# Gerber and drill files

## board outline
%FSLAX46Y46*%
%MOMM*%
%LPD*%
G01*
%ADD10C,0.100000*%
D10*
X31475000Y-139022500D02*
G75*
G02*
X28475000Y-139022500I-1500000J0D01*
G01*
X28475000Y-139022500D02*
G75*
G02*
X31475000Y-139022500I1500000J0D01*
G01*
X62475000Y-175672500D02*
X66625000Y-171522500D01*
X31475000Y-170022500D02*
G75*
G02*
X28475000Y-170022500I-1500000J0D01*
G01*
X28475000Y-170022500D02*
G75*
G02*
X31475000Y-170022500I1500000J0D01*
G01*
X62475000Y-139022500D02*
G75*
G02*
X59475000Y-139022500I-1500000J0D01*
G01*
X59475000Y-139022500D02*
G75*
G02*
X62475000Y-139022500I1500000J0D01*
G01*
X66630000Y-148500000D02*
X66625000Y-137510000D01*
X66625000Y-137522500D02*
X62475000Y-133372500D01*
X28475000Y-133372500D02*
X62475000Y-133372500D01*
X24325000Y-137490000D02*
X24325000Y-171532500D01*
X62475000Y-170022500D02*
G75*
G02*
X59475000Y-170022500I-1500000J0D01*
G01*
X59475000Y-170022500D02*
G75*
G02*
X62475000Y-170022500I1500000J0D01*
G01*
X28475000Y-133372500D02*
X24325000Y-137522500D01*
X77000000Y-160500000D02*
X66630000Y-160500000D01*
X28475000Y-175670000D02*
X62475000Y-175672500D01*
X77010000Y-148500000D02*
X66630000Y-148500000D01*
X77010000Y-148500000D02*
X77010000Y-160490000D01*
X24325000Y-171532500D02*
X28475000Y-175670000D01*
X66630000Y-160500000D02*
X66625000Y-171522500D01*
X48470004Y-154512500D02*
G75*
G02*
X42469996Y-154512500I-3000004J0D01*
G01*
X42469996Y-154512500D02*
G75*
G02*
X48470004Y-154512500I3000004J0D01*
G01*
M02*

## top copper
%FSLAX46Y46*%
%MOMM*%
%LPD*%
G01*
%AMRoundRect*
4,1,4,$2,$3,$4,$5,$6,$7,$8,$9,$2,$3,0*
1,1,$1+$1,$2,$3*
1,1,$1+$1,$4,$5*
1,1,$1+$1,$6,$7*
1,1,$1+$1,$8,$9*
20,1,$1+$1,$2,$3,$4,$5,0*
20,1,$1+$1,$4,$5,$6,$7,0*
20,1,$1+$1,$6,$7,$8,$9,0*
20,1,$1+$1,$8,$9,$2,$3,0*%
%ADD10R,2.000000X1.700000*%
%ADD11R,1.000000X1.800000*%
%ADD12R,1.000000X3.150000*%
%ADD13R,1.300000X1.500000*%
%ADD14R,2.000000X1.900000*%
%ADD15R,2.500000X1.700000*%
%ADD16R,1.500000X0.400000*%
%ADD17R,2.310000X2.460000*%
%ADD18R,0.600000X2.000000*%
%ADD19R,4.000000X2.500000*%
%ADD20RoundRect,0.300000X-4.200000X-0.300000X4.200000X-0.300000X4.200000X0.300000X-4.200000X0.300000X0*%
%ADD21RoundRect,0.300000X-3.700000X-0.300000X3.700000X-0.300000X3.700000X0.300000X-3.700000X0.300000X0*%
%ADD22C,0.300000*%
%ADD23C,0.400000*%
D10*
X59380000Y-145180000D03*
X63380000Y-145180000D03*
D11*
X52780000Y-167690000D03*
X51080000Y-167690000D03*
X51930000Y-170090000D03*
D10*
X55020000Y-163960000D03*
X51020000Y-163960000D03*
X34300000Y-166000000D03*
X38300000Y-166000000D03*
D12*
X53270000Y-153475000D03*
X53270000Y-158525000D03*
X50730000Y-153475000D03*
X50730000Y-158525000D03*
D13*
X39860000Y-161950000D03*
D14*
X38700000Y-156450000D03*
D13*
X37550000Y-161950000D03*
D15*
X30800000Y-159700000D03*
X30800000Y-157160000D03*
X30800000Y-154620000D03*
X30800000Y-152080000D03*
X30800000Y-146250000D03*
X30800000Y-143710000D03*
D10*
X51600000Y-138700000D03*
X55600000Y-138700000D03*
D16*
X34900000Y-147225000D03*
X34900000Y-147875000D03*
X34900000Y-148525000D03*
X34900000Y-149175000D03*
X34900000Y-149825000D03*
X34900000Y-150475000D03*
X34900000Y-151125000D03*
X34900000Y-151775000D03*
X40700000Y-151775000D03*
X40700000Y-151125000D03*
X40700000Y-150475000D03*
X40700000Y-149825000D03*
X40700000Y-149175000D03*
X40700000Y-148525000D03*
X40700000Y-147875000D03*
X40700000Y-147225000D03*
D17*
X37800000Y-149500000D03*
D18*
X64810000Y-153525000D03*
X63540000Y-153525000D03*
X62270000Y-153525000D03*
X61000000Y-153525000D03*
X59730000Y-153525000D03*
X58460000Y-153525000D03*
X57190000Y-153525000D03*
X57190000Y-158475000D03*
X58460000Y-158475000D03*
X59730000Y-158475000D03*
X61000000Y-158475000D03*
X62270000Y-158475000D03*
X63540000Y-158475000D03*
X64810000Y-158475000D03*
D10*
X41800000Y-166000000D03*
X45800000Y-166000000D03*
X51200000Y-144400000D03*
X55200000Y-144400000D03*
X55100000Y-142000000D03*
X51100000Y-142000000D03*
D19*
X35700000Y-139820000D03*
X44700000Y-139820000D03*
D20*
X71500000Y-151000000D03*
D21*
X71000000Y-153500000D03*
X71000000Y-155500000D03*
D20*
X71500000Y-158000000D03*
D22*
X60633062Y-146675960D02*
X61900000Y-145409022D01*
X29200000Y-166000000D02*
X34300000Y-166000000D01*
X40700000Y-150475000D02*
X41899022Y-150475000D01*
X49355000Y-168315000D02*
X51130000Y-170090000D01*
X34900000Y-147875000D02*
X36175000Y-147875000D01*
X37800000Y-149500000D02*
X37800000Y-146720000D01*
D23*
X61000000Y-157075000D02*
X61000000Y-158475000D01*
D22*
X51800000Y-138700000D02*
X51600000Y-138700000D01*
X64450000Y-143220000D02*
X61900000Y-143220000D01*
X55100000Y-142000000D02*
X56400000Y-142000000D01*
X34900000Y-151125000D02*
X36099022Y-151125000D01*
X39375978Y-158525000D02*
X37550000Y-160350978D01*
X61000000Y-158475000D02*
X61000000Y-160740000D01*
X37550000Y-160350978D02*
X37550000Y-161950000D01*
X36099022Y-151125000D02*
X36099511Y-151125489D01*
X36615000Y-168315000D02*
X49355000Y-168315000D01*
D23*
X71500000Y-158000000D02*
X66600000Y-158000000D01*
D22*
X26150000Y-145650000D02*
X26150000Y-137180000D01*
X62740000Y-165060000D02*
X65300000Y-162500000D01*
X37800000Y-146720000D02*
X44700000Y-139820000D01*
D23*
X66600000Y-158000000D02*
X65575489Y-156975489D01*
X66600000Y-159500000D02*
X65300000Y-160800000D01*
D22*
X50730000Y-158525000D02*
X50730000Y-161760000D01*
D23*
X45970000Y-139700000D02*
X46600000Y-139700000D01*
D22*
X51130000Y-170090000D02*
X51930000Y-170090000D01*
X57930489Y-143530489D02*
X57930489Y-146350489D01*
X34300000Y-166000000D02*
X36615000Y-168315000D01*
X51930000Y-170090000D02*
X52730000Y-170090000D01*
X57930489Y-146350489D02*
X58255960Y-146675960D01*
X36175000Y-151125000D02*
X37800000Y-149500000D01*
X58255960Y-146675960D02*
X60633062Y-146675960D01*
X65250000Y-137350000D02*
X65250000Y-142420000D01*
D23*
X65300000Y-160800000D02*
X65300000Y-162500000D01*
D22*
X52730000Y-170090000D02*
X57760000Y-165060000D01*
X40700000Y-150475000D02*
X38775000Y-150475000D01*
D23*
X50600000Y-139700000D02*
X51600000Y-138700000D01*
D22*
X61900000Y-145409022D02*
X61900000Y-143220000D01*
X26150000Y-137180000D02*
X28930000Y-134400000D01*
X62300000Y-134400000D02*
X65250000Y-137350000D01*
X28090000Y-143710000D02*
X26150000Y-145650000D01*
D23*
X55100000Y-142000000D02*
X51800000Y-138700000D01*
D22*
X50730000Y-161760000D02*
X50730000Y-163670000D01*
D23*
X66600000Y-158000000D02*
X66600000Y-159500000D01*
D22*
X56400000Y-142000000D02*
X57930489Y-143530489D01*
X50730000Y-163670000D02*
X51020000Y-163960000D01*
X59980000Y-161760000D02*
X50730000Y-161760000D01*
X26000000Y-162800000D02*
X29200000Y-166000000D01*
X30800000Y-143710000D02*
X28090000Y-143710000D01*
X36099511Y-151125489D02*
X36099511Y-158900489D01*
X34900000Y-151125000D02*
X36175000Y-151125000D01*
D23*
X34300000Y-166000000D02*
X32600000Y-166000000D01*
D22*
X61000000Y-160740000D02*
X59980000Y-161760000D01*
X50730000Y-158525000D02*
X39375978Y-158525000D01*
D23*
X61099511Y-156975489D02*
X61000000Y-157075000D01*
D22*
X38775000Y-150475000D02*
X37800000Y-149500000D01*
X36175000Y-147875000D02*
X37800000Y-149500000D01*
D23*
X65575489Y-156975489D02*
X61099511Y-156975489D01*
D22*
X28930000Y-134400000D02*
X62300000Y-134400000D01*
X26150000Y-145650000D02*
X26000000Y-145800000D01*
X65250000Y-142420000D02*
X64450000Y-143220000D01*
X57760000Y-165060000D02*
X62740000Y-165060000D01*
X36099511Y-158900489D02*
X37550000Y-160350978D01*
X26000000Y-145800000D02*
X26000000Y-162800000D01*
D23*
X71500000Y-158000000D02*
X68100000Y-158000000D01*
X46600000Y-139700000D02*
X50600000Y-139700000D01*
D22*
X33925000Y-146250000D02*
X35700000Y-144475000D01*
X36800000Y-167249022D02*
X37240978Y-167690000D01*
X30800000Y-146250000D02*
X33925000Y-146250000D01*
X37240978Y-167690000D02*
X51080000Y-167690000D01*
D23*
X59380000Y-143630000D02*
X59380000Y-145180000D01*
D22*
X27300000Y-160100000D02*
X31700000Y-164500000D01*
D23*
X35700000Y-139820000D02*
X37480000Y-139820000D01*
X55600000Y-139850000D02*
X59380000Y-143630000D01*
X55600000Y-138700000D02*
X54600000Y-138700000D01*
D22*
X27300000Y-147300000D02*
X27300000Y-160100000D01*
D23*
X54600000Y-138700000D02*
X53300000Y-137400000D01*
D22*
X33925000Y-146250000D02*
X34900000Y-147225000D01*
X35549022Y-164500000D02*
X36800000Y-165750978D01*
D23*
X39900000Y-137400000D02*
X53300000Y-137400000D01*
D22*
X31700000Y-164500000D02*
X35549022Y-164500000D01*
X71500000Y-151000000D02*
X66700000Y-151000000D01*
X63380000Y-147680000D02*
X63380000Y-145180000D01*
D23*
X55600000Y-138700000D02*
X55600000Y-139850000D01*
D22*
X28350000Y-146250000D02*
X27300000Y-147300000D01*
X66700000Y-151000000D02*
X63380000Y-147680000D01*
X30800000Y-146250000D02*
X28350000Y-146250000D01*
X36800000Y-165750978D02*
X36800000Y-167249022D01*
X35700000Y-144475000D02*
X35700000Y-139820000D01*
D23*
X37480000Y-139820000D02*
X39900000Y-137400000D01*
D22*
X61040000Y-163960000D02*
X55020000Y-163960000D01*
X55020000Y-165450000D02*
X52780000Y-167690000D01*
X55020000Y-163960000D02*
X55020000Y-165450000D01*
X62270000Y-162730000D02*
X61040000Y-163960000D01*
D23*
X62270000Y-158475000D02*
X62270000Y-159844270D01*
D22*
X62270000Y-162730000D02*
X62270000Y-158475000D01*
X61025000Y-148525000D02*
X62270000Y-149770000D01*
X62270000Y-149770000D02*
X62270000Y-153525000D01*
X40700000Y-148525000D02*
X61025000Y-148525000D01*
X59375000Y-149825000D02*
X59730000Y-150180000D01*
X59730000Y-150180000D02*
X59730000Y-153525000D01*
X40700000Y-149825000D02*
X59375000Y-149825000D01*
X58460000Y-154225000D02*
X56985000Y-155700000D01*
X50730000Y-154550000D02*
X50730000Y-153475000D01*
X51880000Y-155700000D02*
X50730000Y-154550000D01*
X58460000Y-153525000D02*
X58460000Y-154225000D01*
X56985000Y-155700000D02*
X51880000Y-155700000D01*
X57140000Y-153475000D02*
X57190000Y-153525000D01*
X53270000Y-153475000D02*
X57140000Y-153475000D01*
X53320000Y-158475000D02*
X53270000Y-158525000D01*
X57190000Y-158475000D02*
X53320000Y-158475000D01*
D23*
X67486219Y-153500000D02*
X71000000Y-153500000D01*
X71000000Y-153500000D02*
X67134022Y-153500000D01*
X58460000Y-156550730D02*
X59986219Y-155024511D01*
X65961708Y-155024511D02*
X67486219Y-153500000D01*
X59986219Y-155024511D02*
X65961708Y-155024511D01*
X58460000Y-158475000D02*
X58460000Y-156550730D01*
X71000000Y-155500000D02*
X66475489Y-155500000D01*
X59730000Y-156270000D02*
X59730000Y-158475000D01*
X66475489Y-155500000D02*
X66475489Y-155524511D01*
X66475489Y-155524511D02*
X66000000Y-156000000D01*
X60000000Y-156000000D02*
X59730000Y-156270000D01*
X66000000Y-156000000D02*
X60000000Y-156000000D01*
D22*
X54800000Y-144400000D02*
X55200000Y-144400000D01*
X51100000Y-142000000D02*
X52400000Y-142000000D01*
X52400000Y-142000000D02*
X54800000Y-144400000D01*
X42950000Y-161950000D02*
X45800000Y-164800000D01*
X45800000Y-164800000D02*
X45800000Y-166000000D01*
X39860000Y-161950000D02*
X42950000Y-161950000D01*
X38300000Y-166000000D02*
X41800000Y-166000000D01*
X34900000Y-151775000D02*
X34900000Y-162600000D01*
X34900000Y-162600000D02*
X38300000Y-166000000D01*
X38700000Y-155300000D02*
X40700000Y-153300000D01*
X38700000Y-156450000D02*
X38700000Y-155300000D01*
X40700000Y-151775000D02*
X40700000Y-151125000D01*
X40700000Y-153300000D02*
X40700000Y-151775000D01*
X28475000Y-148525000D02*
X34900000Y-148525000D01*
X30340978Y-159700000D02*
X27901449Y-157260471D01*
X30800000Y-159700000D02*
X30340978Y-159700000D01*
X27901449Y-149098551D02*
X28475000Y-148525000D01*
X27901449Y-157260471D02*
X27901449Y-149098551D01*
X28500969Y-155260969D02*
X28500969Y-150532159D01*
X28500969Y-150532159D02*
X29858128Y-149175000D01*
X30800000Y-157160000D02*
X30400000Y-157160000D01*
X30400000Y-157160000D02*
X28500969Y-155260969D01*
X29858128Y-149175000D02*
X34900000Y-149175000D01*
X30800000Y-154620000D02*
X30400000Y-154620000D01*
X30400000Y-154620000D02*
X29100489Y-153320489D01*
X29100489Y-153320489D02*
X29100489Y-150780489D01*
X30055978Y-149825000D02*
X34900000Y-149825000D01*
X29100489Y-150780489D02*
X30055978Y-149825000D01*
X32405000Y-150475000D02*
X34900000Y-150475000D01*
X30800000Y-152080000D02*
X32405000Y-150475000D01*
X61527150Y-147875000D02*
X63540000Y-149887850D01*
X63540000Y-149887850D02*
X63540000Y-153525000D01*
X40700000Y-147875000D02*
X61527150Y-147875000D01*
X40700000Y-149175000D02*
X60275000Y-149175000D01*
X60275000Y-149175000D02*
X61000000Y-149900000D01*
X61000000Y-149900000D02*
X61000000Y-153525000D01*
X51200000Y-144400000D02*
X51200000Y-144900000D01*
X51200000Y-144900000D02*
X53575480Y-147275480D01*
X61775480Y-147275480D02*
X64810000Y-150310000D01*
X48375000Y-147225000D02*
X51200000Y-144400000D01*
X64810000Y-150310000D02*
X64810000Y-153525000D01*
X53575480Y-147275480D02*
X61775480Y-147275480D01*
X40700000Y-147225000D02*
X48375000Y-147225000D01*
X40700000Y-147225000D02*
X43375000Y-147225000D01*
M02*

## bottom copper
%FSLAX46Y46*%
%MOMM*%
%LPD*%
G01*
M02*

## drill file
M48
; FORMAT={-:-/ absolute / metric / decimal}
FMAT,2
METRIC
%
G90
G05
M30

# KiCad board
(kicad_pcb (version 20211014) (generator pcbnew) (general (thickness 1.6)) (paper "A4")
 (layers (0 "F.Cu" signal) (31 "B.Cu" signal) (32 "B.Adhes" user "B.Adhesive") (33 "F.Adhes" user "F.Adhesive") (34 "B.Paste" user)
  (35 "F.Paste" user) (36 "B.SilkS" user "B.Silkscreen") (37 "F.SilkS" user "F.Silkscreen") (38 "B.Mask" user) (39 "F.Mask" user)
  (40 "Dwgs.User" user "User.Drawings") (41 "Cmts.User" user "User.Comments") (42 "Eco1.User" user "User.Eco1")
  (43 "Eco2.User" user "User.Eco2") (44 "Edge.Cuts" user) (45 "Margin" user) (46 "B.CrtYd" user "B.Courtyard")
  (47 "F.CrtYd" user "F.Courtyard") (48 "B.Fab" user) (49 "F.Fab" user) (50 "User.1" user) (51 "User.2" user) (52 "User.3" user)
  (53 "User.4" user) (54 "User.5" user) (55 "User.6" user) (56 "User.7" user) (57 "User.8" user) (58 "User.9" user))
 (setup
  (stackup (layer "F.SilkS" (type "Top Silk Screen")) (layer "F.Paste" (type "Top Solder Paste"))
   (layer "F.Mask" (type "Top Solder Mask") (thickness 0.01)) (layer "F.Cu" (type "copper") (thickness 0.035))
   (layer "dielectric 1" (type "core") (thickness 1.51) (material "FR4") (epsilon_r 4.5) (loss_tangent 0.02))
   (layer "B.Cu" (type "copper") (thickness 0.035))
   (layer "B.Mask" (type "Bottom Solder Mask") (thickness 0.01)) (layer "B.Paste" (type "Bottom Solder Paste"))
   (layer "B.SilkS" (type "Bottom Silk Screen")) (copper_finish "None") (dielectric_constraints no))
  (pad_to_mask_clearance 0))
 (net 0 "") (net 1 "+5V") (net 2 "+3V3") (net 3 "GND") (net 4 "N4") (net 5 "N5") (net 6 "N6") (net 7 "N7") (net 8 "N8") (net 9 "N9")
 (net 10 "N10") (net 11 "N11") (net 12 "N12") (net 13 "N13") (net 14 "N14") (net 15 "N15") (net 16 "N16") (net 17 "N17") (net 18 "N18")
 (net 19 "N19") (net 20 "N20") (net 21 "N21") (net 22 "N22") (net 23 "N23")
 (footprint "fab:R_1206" (layer "F.Cu") (at 61.38 145.18)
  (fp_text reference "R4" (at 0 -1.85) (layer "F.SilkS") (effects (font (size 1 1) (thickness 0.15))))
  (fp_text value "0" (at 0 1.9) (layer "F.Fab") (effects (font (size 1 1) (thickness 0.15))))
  (pad "1" smd rect locked (at -2 0) (size 2 1.7) (layers "F.Cu" "F.Paste" "F.Mask") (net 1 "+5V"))
  (pad "2" smd rect locked (at 2 0) (size 2 1.7) (layers "F.Cu" "F.Paste" "F.Mask") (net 1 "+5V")))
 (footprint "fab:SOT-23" (layer "F.Cu") (at 51.93 168.89 -90)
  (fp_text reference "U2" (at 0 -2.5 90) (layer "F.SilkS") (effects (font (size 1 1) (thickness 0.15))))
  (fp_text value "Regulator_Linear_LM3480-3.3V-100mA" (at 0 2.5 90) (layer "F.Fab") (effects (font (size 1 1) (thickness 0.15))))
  (pad "1" smd rect locked (at -1.2 -0.85 270) (size 1.8 1) (layers "F.Cu" "F.Paste" "F.Mask") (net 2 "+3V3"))
  (pad "2" smd rect locked (at -1.2 0.85 270) (size 1.8 1) (layers "F.Cu" "F.Paste" "F.Mask") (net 1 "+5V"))
  (pad "3" smd rect locked (at 1.2 0 270) (size 1.8 1) (layers "F.Cu" "F.Paste" "F.Mask") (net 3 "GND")))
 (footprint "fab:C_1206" (layer "F.Cu") (at 53.02 163.96 180)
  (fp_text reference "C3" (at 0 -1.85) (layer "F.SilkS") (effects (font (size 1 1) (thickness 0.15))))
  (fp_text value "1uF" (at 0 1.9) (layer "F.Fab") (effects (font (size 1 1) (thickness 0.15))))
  (pad "1" smd rect locked (at -2 0 180) (size 2 1.7) (layers "F.Cu" "F.Paste" "F.Mask") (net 2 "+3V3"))
  (pad "2" smd rect locked (at 2 0 180) (size 2 1.7) (layers "F.Cu" "F.Paste" "F.Mask") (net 3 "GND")))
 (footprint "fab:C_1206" (layer "F.Cu") (at 36.3 166)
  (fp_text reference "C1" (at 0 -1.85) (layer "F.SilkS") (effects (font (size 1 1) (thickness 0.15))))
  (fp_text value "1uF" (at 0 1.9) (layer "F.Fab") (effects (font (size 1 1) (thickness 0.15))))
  (pad "1" smd rect locked (at -2 0) (size 2 1.7) (layers "F.Cu" "F.Paste" "F.Mask") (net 3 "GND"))
  (pad "2" smd rect locked (at 2 0) (size 2 1.7) (layers "F.Cu" "F.Paste" "F.Mask") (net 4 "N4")))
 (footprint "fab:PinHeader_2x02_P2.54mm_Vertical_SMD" (layer "F.Cu") (at 52 156 -90)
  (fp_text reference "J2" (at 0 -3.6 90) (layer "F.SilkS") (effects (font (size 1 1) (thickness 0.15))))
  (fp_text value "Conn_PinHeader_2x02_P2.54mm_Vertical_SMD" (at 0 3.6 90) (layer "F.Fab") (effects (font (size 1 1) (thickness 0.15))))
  (pad "1" smd rect locked (at -2.525 -1.27 270) (size 3.15 1) (layers "F.Cu" "F.Paste" "F.Mask") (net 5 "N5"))
  (pad "2" smd rect locked (at 2.525 -1.27 270) (size 3.15 1) (layers "F.Cu" "F.Paste" "F.Mask") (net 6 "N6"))
  (pad "3" smd rect locked (at -2.525 1.27 270) (size 3.15 1) (layers "F.Cu" "F.Paste" "F.Mask") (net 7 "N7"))
  (pad "4" smd rect locked (at 2.525 1.27 270) (size 3.15 1) (layers "F.Cu" "F.Paste" "F.Mask") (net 3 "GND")))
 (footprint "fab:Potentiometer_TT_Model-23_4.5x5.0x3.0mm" (layer "F.Cu") (at 38.7 159.2)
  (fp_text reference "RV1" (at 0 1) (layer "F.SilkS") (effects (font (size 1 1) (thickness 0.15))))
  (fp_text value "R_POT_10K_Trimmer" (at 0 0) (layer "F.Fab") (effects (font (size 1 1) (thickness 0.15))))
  (pad "1" smd rect locked (at 1.16 2.75) (size 1.3 1.5) (layers "F.Cu" "F.Paste" "F.Mask") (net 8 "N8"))
  (pad "2" smd rect locked (at 0 -2.75) (size 2 1.9) (layers "F.Cu" "F.Paste" "F.Mask") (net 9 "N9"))
  (pad "3" smd rect locked (at -1.15 2.75) (size 1.3 1.5) (layers "F.Cu" "F.Paste" "F.Mask") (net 3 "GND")))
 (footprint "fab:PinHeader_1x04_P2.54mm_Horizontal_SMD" (layer "F.Cu") (at 30.8 159.7 180)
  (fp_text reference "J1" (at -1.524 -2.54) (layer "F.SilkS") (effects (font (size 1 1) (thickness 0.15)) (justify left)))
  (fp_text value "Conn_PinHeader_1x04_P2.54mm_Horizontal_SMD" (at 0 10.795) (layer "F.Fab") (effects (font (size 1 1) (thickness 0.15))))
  (pad "1" smd rect locked (at 0 0 180) (size 2.5 1.7) (layers "F.Cu" "F.Paste" "F.Mask") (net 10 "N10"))
  (pad "2" smd rect locked (at 0 2.54 180) (size 2.5 1.7) (layers "F.Cu" "F.Paste" "F.Mask") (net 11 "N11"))
  (pad "3" smd rect locked (at 0 5.08 180) (size 2.5 1.7) (layers "F.Cu" "F.Paste" "F.Mask") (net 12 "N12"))
  (pad "4" smd rect locked (at 0 7.62 180) (size 2.5 1.7) (layers "F.Cu" "F.Paste" "F.Mask") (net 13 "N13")))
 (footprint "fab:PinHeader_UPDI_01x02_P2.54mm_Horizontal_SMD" (layer "F.Cu") (at 30.8 146.25 180)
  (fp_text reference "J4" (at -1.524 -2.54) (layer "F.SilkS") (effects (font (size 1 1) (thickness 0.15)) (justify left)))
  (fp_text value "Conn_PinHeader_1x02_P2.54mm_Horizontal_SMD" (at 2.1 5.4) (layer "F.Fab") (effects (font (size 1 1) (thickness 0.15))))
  (pad "1" smd rect locked (at 0 0 180) (size 2.5 1.7) (layers "F.Cu" "F.Paste" "F.Mask") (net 1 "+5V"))
  (pad "2" smd rect locked (at 0 2.54 180) (size 2.5 1.7) (layers "F.Cu" "F.Paste" "F.Mask") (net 3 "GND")))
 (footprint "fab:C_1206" (layer "F.Cu") (at 53.6 138.7)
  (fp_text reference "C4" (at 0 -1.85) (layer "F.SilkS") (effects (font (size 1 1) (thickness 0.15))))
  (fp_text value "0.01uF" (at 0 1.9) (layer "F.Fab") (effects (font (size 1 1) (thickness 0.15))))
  (pad "1" smd rect locked (at -2 0) (size 2 1.7) (layers "F.Cu" "F.Paste" "F.Mask") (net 3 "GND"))
  (pad "2" smd rect locked (at 2 0) (size 2 1.7) (layers "F.Cu" "F.Paste" "F.Mask") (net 1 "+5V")))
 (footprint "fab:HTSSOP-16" (layer "F.Cu") (at 37.8 149.5)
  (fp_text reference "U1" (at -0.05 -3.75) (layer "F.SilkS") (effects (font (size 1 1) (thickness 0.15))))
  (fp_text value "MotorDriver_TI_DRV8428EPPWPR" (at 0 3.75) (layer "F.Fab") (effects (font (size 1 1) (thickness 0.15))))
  (pad "1" smd rect locked (at -2.9 -2.275 270) (size 0.4 1.5) (layers "F.Cu" "F.Paste" "F.Mask") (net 1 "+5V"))
  (pad "2" smd rect locked (at -2.9 -1.625 270) (size 0.4 1.5) (layers "F.Cu" "F.Paste" "F.Mask") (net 3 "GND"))
  (pad "3" smd rect locked (at -2.9 -0.975 270) (size 0.4 1.5) (layers "F.Cu" "F.Paste" "F.Mask") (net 10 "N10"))
  (pad "4" smd rect locked (at -2.9 -0.325 270) (size 0.4 1.5) (layers "F.Cu" "F.Paste" "F.Mask") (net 11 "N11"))
  (pad "5" smd rect locked (at -2.9 0.325 270) (size 0.4 1.5) (layers "F.Cu" "F.Paste" "F.Mask") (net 12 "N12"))
  (pad "6" smd rect locked (at -2.9 0.975 270) (size 0.4 1.5) (layers "F.Cu" "F.Paste" "F.Mask") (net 13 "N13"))
  (pad "7" smd rect locked (at -2.9 1.625 270) (size 0.4 1.5) (layers "F.Cu" "F.Paste" "F.Mask") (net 3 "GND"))
  (pad "8" smd rect locked (at -2.9 2.275 270) (size 0.4 1.5) (layers "F.Cu" "F.Paste" "F.Mask") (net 4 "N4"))
  (pad "9" smd rect locked (at 2.9 2.275 270) (size 0.4 1.5) (layers "F.Cu" "F.Paste" "F.Mask") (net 9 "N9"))
  (pad "10" smd rect locked (at 2.9 1.625 270) (size 0.4 1.5) (layers "F.Cu" "F.Paste" "F.Mask") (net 9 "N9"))
  (pad "11" smd rect locked (at 2.9 0.975 270) (size 0.4 1.5) (layers "F.Cu" "F.Paste" "F.Mask") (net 3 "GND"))
  (pad "12" smd rect locked (at 2.9 0.325 270) (size 0.4 1.5) (layers "F.Cu" "F.Paste" "F.Mask") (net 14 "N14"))
  (pad "13" smd rect locked (at 2.9 -0.325 270) (size 0.4 1.5) (layers "F.Cu" "F.Paste" "F.Mask") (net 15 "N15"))
  (pad "14" smd rect locked (at 2.9 -0.975 270) (size 0.4 1.5) (layers "F.Cu" "F.Paste" "F.Mask") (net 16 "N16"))
  (pad "15" smd rect locked (at 2.9 -1.625 270) (size 0.4 1.5) (layers "F.Cu" "F.Paste" "F.Mask") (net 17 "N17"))
  (pad "16" smd rect locked (at 2.9 -2.275 270) (size 0.4 1.5) (layers "F.Cu" "F.Paste" "F.Mask") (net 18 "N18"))
  (pad "17" smd rect locked (at 0 0 270) (size 2.46 2.31) (layers "F.Cu" "F.Paste" "F.Mask") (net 3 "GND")))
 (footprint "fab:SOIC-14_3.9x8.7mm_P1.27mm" (layer "F.Cu") (at 61 156 -90)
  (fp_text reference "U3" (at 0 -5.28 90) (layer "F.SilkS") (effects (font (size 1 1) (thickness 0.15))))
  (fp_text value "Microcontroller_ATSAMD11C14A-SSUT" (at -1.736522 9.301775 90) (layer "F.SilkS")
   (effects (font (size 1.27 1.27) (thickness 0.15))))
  (pad "1" smd rect locked (at -2.475 -3.81 270) (size 2 0.6) (layers "F.Cu" "F.Paste" "F.Mask") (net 18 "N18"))
  (pad "2" smd rect locked (at -2.475 -2.54 270) (size 2 0.6) (layers "F.Cu" "F.Paste" "F.Mask") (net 17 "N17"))
  (pad "3" smd rect locked (at -2.475 -1.27 270) (size 2 0.6) (layers "F.Cu" "F.Paste" "F.Mask") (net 16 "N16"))
  (pad "4" smd rect locked (at -2.475 0 270) (size 2 0.6) (layers "F.Cu" "F.Paste" "F.Mask") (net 15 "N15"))
  (pad "5" smd rect locked (at -2.475 1.27 270) (size 2 0.6) (layers "F.Cu" "F.Paste" "F.Mask") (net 14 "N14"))
  (pad "6" smd rect locked (at -2.475 2.54 270) (size 2 0.6) (layers "F.Cu" "F.Paste" "F.Mask") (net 7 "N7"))
  (pad "7" smd rect locked (at -2.475 3.81 270) (size 2 0.6) (layers "F.Cu" "F.Paste" "F.Mask") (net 5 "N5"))
  (pad "8" smd rect locked (at 2.475 3.81 270) (size 2 0.6) (layers "F.Cu" "F.Paste" "F.Mask") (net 6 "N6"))
  (pad "9" smd rect locked (at 2.475 2.54 270) (size 2 0.6) (layers "F.Cu" "F.Paste" "F.Mask") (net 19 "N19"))
  (pad "10" smd rect locked (at 2.475 1.27 270) (size 2 0.6) (layers "F.Cu" "F.Paste" "F.Mask") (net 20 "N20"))
  (pad "11" smd rect locked (at 2.475 0 270) (size 2 0.6) (layers "F.Cu" "F.Paste" "F.Mask") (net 3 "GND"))
  (pad "12" smd rect locked (at 2.475 -1.27 270) (size 2 0.6) (layers "F.Cu" "F.Paste" "F.Mask") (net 2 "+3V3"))
  (pad "13" smd rect locked (at 2.475 -2.54 270) (size 2 0.6) (layers "F.Cu" "F.Paste" "F.Mask") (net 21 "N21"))
  (pad "14" smd rect locked (at 2.475 -3.81 270) (size 2 0.6) (layers "F.Cu" "F.Paste" "F.Mask") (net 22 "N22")))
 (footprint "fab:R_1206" (layer "F.Cu") (at 43.8 166)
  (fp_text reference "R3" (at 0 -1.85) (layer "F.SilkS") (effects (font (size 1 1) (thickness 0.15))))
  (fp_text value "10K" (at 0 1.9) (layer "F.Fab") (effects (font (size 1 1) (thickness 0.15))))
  (pad "1" smd rect locked (at -2 0) (size 2 1.7) (layers "F.Cu" "F.Paste" "F.Mask") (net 4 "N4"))
  (pad "2" smd rect locked (at 2 0) (size 2 1.7) (layers "F.Cu" "F.Paste" "F.Mask") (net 8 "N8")))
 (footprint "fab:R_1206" (layer "F.Cu") (at 53.2 144.4)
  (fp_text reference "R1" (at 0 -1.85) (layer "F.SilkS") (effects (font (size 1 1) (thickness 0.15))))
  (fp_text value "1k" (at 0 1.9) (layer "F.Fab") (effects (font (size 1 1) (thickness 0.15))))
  (pad "1" smd rect locked (at -2 0) (size 2 1.7) (layers "F.Cu" "F.Paste" "F.Mask") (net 18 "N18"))
  (pad "2" smd rect locked (at 2 0) (size 2 1.7) (layers "F.Cu" "F.Paste" "F.Mask") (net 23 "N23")))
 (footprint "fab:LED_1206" (layer "F.Cu") (at 53.1 142 180)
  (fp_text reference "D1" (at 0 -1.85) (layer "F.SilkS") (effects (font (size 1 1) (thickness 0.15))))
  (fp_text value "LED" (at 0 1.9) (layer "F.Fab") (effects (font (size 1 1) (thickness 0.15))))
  (pad "1" smd rect locked (at -2 0 180) (size 2 1.7) (layers "F.Cu" "F.Paste" "F.Mask") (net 3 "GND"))
  (pad "2" smd rect locked (at 2 0 180) (size 2 1.7) (layers "F.Cu" "F.Paste" "F.Mask") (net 23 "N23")))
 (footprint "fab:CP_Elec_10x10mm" (layer "F.Cu") (at 40.2 139.82)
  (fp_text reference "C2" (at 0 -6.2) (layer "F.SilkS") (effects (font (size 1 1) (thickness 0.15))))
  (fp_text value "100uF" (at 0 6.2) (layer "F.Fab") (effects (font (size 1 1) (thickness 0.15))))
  (pad "1" smd rect locked (at -4.5 0) (size 4 2.5) (layers "F.Cu" "F.Paste" "F.Mask") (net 1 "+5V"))
  (pad "2" smd rect locked (at 4.5 0) (size 4 2.5) (layers "F.Cu" "F.Paste" "F.Mask") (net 3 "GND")))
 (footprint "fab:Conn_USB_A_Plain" (layer "F.Cu") (at 71 154.5)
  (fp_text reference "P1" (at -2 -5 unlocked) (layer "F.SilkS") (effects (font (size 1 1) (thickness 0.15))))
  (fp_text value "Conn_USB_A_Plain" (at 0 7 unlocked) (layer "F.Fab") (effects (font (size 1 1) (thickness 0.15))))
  (pad "1" smd roundrect (at 0.5 -3.5) (size 9 1.2) (layers "F.Cu" "F.Paste" "F.Mask") (roundrect_rratio 0.25) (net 1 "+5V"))
  (pad "2" smd roundrect (at 0 -1) (size 8 1.2) (layers "F.Cu" "F.Paste" "F.Mask") (roundrect_rratio 0.25) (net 19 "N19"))
  (pad "3" smd roundrect (at 0 1) (size 8 1.2) (layers "F.Cu" "F.Paste" "F.Mask") (roundrect_rratio 0.25) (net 20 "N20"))
  (pad "4" smd roundrect (at 0.5 3.5) (size 9 1.2) (layers "F.Cu" "F.Paste" "F.Mask") (roundrect_rratio 0.25) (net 3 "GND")))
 (gr_circle (center 29.975 139.0225) (end 28.475 139.0225) (layer "Edge.Cuts") (width 0.1) (fill none))
 (gr_line (start 62.475 175.6725) (end 66.625 171.5225) (layer "Edge.Cuts") (width 0.1))
 (gr_circle (center 29.975 170.0225) (end 31.475 170.0225) (layer "Edge.Cuts") (width 0.1) (fill none))
 (gr_circle (center 60.975 139.0225) (end 62.475 139.0225) (layer "Edge.Cuts") (width 0.1) (fill none))
 (gr_line (start 66.63 148.5) (end 66.625 137.51) (layer "Edge.Cuts") (width 0.1))
 (gr_line (start 66.625 137.5225) (end 62.475 133.3725) (layer "Edge.Cuts") (width 0.1))
 (gr_line (start 28.475 133.3725) (end 62.475 133.3725) (layer "Edge.Cuts") (width 0.1))
 (gr_line (start 24.325 137.49) (end 24.325 171.5325) (layer "Edge.Cuts") (width 0.1))
 (gr_circle (center 60.975 170.0225) (end 62.475 170.0225) (layer "Edge.Cuts") (width 0.1) (fill none))
 (gr_line (start 28.475 133.3725) (end 24.325 137.5225) (layer "Edge.Cuts") (width 0.1))
 (gr_line (start 77 160.5) (end 66.63 160.5) (layer "Edge.Cuts") (width 0.1))
 (gr_line (start 28.475 175.67) (end 62.475 175.6725) (layer "Edge.Cuts") (width 0.1))
 (gr_line (start 77.01 148.5) (end 66.63 148.5) (layer "Edge.Cuts") (width 0.1))
 (gr_line (start 77.01 148.5) (end 77.01 160.49) (layer "Edge.Cuts") (width 0.1))
 (gr_line (start 24.325 171.5325) (end 28.475 175.67) (layer "Edge.Cuts") (width 0.1))
 (gr_line (start 66.63 160.5) (end 66.625 171.5225) (layer "Edge.Cuts") (width 0.1))
 (gr_circle (center 45.47 154.5125) (end 45.475 151.5125) (layer "Edge.Cuts") (width 0.1) (fill none))
 (segment (start 60.633062 146.67596) (end 61.9 145.409022) (width 0.3) (layer "F.Cu") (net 3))
 (segment (start 29.2 166) (end 34.3 166) (width 0.3) (layer "F.Cu") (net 3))
 (segment (start 40.7 150.475) (end 41.899022 150.475) (width 0.3) (layer "F.Cu") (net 3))
 (segment (start 49.355 168.315) (end 51.13 170.09) (width 0.3) (layer "F.Cu") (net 3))
 (segment (start 34.9 147.875) (end 36.175 147.875) (width 0.3) (layer "F.Cu") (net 3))
 (segment (start 37.8 149.5) (end 37.8 146.72) (width 0.3) (layer "F.Cu") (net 3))
 (segment (start 61 157.075) (end 61 158.475) (width 0.4) (layer "F.Cu") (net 3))
 (segment (start 51.8 138.7) (end 51.6 138.7) (width 0.3) (layer "F.Cu") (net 3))
 (segment (start 64.45 143.22) (end 61.9 143.22) (width 0.3) (layer "F.Cu") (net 3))
 (segment (start 55.1 142) (end 56.4 142) (width 0.3) (layer "F.Cu") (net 3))
 (segment (start 34.9 151.125) (end 36.099022 151.125) (width 0.3) (layer "F.Cu") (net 3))
 (segment (start 39.375978 158.525) (end 37.55 160.350978) (width 0.3) (layer "F.Cu") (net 3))
 (segment (start 61 158.475) (end 61 160.74) (width 0.3) (layer "F.Cu") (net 3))
 (segment (start 37.55 160.350978) (end 37.55 161.95) (width 0.3) (layer "F.Cu") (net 3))
 (segment (start 36.099022 151.125) (end 36.099511 151.125489) (width 0.3) (layer "F.Cu") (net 3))
 (segment (start 36.615 168.315) (end 49.355 168.315) (width 0.3) (layer "F.Cu") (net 3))
 (segment (start 71.5 158) (end 66.6 158) (width 0.4) (layer "F.Cu") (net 3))
 (segment (start 26.15 145.65) (end 26.15 137.18) (width 0.3) (layer "F.Cu") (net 3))
 (segment (start 62.74 165.06) (end 65.3 162.5) (width 0.3) (layer "F.Cu") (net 3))
 (segment (start 37.8 146.72) (end 44.7 139.82) (width 0.3) (layer "F.Cu") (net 3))
 (segment (start 66.6 158) (end 65.575489 156.975489) (width 0.4) (layer "F.Cu") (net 3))
 (segment (start 66.6 159.5) (end 65.3 160.8) (width 0.4) (layer "F.Cu") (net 3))
 (segment (start 50.73 158.525) (end 50.73 161.76) (width 0.3) (layer "F.Cu") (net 3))
 (segment (start 45.97 139.7) (end 46.6 139.7) (width 0.4) (layer "F.Cu") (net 3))
 (segment (start 51.13 170.09) (end 51.93 170.09) (width 0.3) (layer "F.Cu") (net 3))
 (segment (start 57.930489 143.530489) (end 57.930489 146.350489) (width 0.3) (layer "F.Cu") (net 3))
 (segment (start 34.3 166) (end 36.615 168.315) (width 0.3) (layer "F.Cu") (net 3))
 (segment (start 51.93 170.09) (end 52.73 170.09) (width 0.3) (layer "F.Cu") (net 3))
 (segment (start 57.930489 146.350489) (end 58.25596 146.67596) (width 0.3) (layer "F.Cu") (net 3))
 (segment (start 36.175 151.125) (end 37.8 149.5) (width 0.3) (layer "F.Cu") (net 3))
 (segment (start 58.25596 146.67596) (end 60.633062 146.67596) (width 0.3) (layer "F.Cu") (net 3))
 (segment (start 65.25 137.35) (end 65.25 142.42) (width 0.3) (layer "F.Cu") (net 3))
 (segment (start 65.3 160.8) (end 65.3 162.5) (width 0.4) (layer "F.Cu") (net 3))
 (segment (start 52.73 170.09) (end 57.76 165.06) (width 0.3) (layer "F.Cu") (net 3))
 (segment (start 40.7 150.475) (end 38.775 150.475) (width 0.3) (layer "F.Cu") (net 3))
 (segment (start 50.6 139.7) (end 51.6 138.7) (width 0.4) (layer "F.Cu") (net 3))
 (segment (start 61.9 145.409022) (end 61.9 143.22) (width 0.3) (layer "F.Cu") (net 3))
 (segment (start 26.15 137.18) (end 28.93 134.4) (width 0.3) (layer "F.Cu") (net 3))
 (segment (start 62.3 134.4) (end 65.25 137.35) (width 0.3) (layer "F.Cu") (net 3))
 (segment (start 28.09 143.71) (end 26.15 145.65) (width 0.3) (layer "F.Cu") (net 3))
 (segment (start 55.1 142) (end 51.8 138.7) (width 0.4) (layer "F.Cu") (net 3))
 (segment (start 50.73 161.76) (end 50.73 163.67) (width 0.3) (layer "F.Cu") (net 3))
 (segment (start 66.6 158) (end 66.6 159.5) (width 0.4) (layer "F.Cu") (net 3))
 (segment (start 56.4 142) (end 57.930489 143.530489) (width 0.3) (layer "F.Cu") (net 3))
 (segment (start 50.73 163.67) (end 51.02 163.96) (width 0.3) (layer "F.Cu") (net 3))
 (segment (start 59.98 161.76) (end 50.73 161.76) (width 0.3) (layer "F.Cu") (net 3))
 (segment (start 26 162.8) (end 29.2 166) (width 0.3) (layer "F.Cu") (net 3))
 (segment (start 30.8 143.71) (end 28.09 143.71) (width 0.3) (layer "F.Cu") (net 3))
 (segment (start 36.099511 151.125489) (end 36.099511 158.900489) (width 0.3) (layer "F.Cu") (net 3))
 (segment (start 34.9 151.125) (end 36.175 151.125) (width 0.3) (layer "F.Cu") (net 3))
 (segment (start 34.3 166) (end 32.6 166) (width 0.4) (layer "F.Cu") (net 3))
 (segment (start 61 160.74) (end 59.98 161.76) (width 0.3) (layer "F.Cu") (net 3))
 (segment (start 50.73 158.525) (end 39.375978 158.525) (width 0.3) (layer "F.Cu") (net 3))
 (segment (start 61.099511 156.975489) (end 61 157.075) (width 0.4) (layer "F.Cu") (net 3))
 (segment (start 38.775 150.475) (end 37.8 149.5) (width 0.3) (layer "F.Cu") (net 3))
 (segment (start 36.175 147.875) (end 37.8 149.5) (width 0.3) (layer "F.Cu") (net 3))
 (segment (start 65.575489 156.975489) (end 61.099511 156.975489) (width 0.4) (layer "F.Cu") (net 3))
 (segment (start 28.93 134.4) (end 62.3 134.4) (width 0.3) (layer "F.Cu") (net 3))
 (segment (start 26.15 145.65) (end 26 145.8) (width 0.3) (layer "F.Cu") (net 3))
 (segment (start 65.25 142.42) (end 64.45 143.22) (width 0.3) (layer "F.Cu") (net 3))
 (segment (start 57.76 165.06) (end 62.74 165.06) (width 0.3) (layer "F.Cu") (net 3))
 (segment (start 36.099511 158.900489) (end 37.55 160.350978) (width 0.3) (layer "F.Cu") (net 3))
 (segment (start 26 145.8) (end 26 162.8) (width 0.3) (layer "F.Cu") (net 3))
 (segment (start 71.5 158) (end 68.1 158) (width 0.4) (layer "F.Cu") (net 3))
 (segment (start 46.6 139.7) (end 50.6 139.7) (width 0.4) (layer "F.Cu") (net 3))
 (segment (start 33.925 146.25) (end 35.7 144.475) (width 0.3) (layer "F.Cu") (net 1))
 (segment (start 36.8 167.249022) (end 37.240978 167.69) (width 0.3) (layer "F.Cu") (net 1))
 (segment (start 30.8 146.25) (end 33.925 146.25) (width 0.3) (layer "F.Cu") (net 1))
 (segment (start 37.240978 167.69) (end 51.08 167.69) (width 0.3) (layer "F.Cu") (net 1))
 (segment (start 59.38 143.63) (end 59.38 145.18) (width 0.4) (layer "F.Cu") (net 1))
 (segment (start 27.3 160.1) (end 31.7 164.5) (width 0.3) (layer "F.Cu") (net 1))
 (segment (start 35.7 139.82) (end 37.48 139.82) (width 0.4) (layer "F.Cu") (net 1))
 (segment (start 55.6 139.85) (end 59.38 143.63) (width 0.4) (layer "F.Cu") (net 1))
 (segment (start 55.6 138.7) (end 54.6 138.7) (width 0.4) (layer "F.Cu") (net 1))
 (segment (start 27.3 147.3) (end 27.3 160.1) (width 0.3) (layer "F.Cu") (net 1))
 (segment (start 54.6 138.7) (end 53.3 137.4) (width 0.4) (layer "F.Cu") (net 1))
 (segment (start 33.925 146.25) (end 34.9 147.225) (width 0.3) (layer "F.Cu") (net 1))
 (segment (start 35.549022 164.5) (end 36.8 165.750978) (width 0.3) (layer "F.Cu") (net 1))
 (segment (start 39.9 137.4) (end 53.3 137.4) (width 0.4) (layer "F.Cu") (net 1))
 (segment (start 31.7 164.5) (end 35.549022 164.5) (width 0.3) (layer "F.Cu") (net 1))
 (segment (start 71.5 151) (end 66.7 151) (width 0.3) (layer "F.Cu") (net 1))
 (segment (start 63.38 147.68) (end 63.38 145.18) (width 0.3) (layer "F.Cu") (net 1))
 (segment (start 55.6 138.7) (end 55.6 139.85) (width 0.4) (layer "F.Cu") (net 1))
 (segment (start 28.35 146.25) (end 27.3 147.3) (width 0.3) (layer "F.Cu") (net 1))
 (segment (start 66.7 151) (end 63.38 147.68) (width 0.3) (layer "F.Cu") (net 1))
 (segment (start 30.8 146.25) (end 28.35 146.25) (width 0.3) (layer "F.Cu") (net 1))
 (segment (start 36.8 165.750978) (end 36.8 167.249022) (width 0.3) (layer "F.Cu") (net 1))
 (segment (start 35.7 144.475) (end 35.7 139.82) (width 0.3) (layer "F.Cu") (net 1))
 (segment (start 37.48 139.82) (end 39.9 137.4) (width 0.4) (layer "F.Cu") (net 1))
 (segment (start 61.04 163.96) (end 55.02 163.96) (width 0.3) (layer "F.Cu") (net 2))
 (segment (start 55.02 165.45) (end 52.78 167.69) (width 0.3) (layer "F.Cu") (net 2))
 (segment (start 55.02 163.96) (end 55.02 165.45) (width 0.3) (layer "F.Cu") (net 2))
 (segment (start 62.27 162.73) (end 61.04 163.96) (width 0.3) (layer "F.Cu") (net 2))
 (segment (start 62.27 158.475) (end 62.27 159.84427) (width 0.4) (layer "F.Cu") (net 2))
 (segment (start 62.27 162.73) (end 62.27 158.475) (width 0.3) (layer "F.Cu") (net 2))
 (segment (start 61.025 148.525) (end 62.27 149.77) (width 0.3) (layer "F.Cu") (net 16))
 (segment (start 62.27 149.77) (end 62.27 153.525) (width 0.3) (layer "F.Cu") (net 16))
 (segment (start 40.7 148.525) (end 61.025 148.525) (width 0.3) (layer "F.Cu") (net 16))
 (segment (start 59.375 149.825) (end 59.73 150.18) (width 0.3) (layer "F.Cu") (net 14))
 (segment (start 59.73 150.18) (end 59.73 153.525) (width 0.3) (layer "F.Cu") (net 14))
 (segment (start 40.7 149.825) (end 59.375 149.825) (width 0.3) (layer "F.Cu") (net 14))
 (segment (start 58.46 154.225) (end 56.985 155.7) (width 0.3) (layer "F.Cu") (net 7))
 (segment (start 50.73 154.55) (end 50.73 153.475) (width 0.3) (layer "F.Cu") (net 7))
 (segment (start 51.88 155.7) (end 50.73 154.55) (width 0.3) (layer "F.Cu") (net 7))
 (segment (start 58.46 153.525) (end 58.46 154.225) (width 0.3) (layer "F.Cu") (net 7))
 (segment (start 56.985 155.7) (end 51.88 155.7) (width 0.3) (layer "F.Cu") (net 7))
 (segment (start 57.14 153.475) (end 57.19 153.525) (width 0.3) (layer "F.Cu") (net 5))
 (segment (start 53.27 153.475) (end 57.14 153.475) (width 0.3) (layer "F.Cu") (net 5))
 (segment (start 53.32 158.475) (end 53.27 158.525) (width 0.3) (layer "F.Cu") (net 6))
 (segment (start 57.19 158.475) (end 53.32 158.475) (width 0.3) (layer "F.Cu") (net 6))
 (segment (start 67.486219 153.5) (end 71 153.5) (width 0.4) (layer "F.Cu") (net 19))
 (segment (start 71 153.5) (end 67.134022 153.5) (width 0.4) (layer "F.Cu") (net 19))
 (segment (start 58.46 156.55073) (end 59.986219 155.024511) (width 0.4) (layer "F.Cu") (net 19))
 (segment (start 65.961708 155.024511) (end 67.486219 153.5) (width 0.4) (layer "F.Cu") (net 19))
 (segment (start 59.986219 155.024511) (end 65.961708 155.024511) (width 0.4) (layer "F.Cu") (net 19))
 (segment (start 58.46 158.475) (end 58.46 156.55073) (width 0.4) (layer "F.Cu") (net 19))
 (segment (start 71 155.5) (end 66.475489 155.5) (width 0.4) (layer "F.Cu") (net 20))
 (segment (start 59.73 156.27) (end 59.73 158.475) (width 0.4) (layer "F.Cu") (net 20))
 (segment (start 66.475489 155.5) (end 66.475489 155.524511) (width 0.4) (layer "F.Cu") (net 20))
 (segment (start 66.475489 155.524511) (end 66 156) (width 0.4) (layer "F.Cu") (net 20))
 (segment (start 60 156) (end 59.73 156.27) (width 0.4) (layer "F.Cu") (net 20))
 (segment (start 66 156) (end 60 156) (width 0.4) (layer "F.Cu") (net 20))
 (segment (start 54.8 144.4) (end 55.2 144.4) (width 0.3) (layer "F.Cu") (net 23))
 (segment (start 51.1 142) (end 52.4 142) (width 0.3) (layer "F.Cu") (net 23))
 (segment (start 52.4 142) (end 54.8 144.4) (width 0.3) (layer "F.Cu") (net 23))
 (segment (start 42.95 161.95) (end 45.8 164.8) (width 0.3) (layer "F.Cu") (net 8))
 (segment (start 45.8 164.8) (end 45.8 166) (width 0.3) (layer "F.Cu") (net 8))
 (segment (start 39.86 161.95) (end 42.95 161.95) (width 0.3) (layer "F.Cu") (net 8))
 (segment (start 38.3 166) (end 41.8 166) (width 0.3) (layer "F.Cu") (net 4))
 (segment (start 34.9 151.775) (end 34.9 162.6) (width 0.3) (layer "F.Cu") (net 4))
 (segment (start 34.9 162.6) (end 38.3 166) (width 0.3) (layer "F.Cu") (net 4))
 (segment (start 38.7 155.3) (end 40.7 153.3) (width 0.3) (layer "F.Cu") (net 9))
 (segment (start 38.7 156.45) (end 38.7 155.3) (width 0.3) (layer "F.Cu") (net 9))
 (segment (start 40.7 151.775) (end 40.7 151.125) (width 0.3) (layer "F.Cu") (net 9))
 (segment (start 40.7 153.3) (end 40.7 151.775) (width 0.3) (layer "F.Cu") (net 9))
 (segment (start 28.475 148.525) (end 34.9 148.525) (width 0.3) (layer "F.Cu") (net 10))
 (segment (start 30.340978 159.7) (end 27.901449 157.260471) (width 0.3) (layer "F.Cu") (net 10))
 (segment (start 30.8 159.7) (end 30.340978 159.7) (width 0.3) (layer "F.Cu") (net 10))
 (segment (start 27.901449 149.098551) (end 28.475 148.525) (width 0.3) (layer "F.Cu") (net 10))
 (segment (start 27.901449 157.260471) (end 27.901449 149.098551) (width 0.3) (layer "F.Cu") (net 10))
 (segment (start 28.500969 155.260969) (end 28.500969 150.532159) (width 0.3) (layer "F.Cu") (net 11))
 (segment (start 28.500969 150.532159) (end 29.858128 149.175) (width 0.3) (layer "F.Cu") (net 11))
 (segment (start 30.8 157.16) (end 30.4 157.16) (width 0.3) (layer "F.Cu") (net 11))
 (segment (start 30.4 157.16) (end 28.500969 155.260969) (width 0.3) (layer "F.Cu") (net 11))
 (segment (start 29.858128 149.175) (end 34.9 149.175) (width 0.3) (layer "F.Cu") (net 11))
 (segment (start 30.8 154.62) (end 30.4 154.62) (width 0.3) (layer "F.Cu") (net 12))
 (segment (start 30.4 154.62) (end 29.100489 153.320489) (width 0.3) (layer "F.Cu") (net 12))
 (segment (start 29.100489 153.320489) (end 29.100489 150.780489) (width 0.3) (layer "F.Cu") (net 12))
 (segment (start 30.055978 149.825) (end 34.9 149.825) (width 0.3) (layer "F.Cu") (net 12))
 (segment (start 29.100489 150.780489) (end 30.055978 149.825) (width 0.3) (layer "F.Cu") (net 12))
 (segment (start 32.405 150.475) (end 34.9 150.475) (width 0.3) (layer "F.Cu") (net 13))
 (segment (start 30.8 152.08) (end 32.405 150.475) (width 0.3) (layer "F.Cu") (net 13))
 (segment (start 61.52715 147.875) (end 63.54 149.88785) (width 0.3) (layer "F.Cu") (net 17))
 (segment (start 63.54 149.88785) (end 63.54 153.525) (width 0.3) (layer "F.Cu") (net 17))
 (segment (start 40.7 147.875) (end 61.52715 147.875) (width 0.3) (layer "F.Cu") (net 17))
 (segment (start 40.7 149.175) (end 60.275 149.175) (width 0.3) (layer "F.Cu") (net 15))
 (segment (start 60.275 149.175) (end 61 149.9) (width 0.3) (layer "F.Cu") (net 15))
 (segment (start 61 149.9) (end 61 153.525) (width 0.3) (layer "F.Cu") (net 15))
 (segment (start 51.2 144.4) (end 51.2 144.9) (width 0.3) (layer "F.Cu") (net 18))
 (segment (start 51.2 144.9) (end 53.57548 147.27548) (width 0.3) (layer "F.Cu") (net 18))
 (segment (start 61.77548 147.27548) (end 64.81 150.31) (width 0.3) (layer "F.Cu") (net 18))
 (segment (start 48.375 147.225) (end 51.2 144.4) (width 0.3) (layer "F.Cu") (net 18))
 (segment (start 64.81 150.31) (end 64.81 153.525) (width 0.3) (layer "F.Cu") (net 18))
 (segment (start 53.57548 147.27548) (end 61.77548 147.27548) (width 0.3) (layer "F.Cu") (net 18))
 (segment (start 40.7 147.225) (end 48.375 147.225) (width 0.3) (layer "F.Cu") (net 18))
 (segment (start 40.7 147.225) (end 43.375 147.225) (width 0.3) (layer "F.Cu") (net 18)))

